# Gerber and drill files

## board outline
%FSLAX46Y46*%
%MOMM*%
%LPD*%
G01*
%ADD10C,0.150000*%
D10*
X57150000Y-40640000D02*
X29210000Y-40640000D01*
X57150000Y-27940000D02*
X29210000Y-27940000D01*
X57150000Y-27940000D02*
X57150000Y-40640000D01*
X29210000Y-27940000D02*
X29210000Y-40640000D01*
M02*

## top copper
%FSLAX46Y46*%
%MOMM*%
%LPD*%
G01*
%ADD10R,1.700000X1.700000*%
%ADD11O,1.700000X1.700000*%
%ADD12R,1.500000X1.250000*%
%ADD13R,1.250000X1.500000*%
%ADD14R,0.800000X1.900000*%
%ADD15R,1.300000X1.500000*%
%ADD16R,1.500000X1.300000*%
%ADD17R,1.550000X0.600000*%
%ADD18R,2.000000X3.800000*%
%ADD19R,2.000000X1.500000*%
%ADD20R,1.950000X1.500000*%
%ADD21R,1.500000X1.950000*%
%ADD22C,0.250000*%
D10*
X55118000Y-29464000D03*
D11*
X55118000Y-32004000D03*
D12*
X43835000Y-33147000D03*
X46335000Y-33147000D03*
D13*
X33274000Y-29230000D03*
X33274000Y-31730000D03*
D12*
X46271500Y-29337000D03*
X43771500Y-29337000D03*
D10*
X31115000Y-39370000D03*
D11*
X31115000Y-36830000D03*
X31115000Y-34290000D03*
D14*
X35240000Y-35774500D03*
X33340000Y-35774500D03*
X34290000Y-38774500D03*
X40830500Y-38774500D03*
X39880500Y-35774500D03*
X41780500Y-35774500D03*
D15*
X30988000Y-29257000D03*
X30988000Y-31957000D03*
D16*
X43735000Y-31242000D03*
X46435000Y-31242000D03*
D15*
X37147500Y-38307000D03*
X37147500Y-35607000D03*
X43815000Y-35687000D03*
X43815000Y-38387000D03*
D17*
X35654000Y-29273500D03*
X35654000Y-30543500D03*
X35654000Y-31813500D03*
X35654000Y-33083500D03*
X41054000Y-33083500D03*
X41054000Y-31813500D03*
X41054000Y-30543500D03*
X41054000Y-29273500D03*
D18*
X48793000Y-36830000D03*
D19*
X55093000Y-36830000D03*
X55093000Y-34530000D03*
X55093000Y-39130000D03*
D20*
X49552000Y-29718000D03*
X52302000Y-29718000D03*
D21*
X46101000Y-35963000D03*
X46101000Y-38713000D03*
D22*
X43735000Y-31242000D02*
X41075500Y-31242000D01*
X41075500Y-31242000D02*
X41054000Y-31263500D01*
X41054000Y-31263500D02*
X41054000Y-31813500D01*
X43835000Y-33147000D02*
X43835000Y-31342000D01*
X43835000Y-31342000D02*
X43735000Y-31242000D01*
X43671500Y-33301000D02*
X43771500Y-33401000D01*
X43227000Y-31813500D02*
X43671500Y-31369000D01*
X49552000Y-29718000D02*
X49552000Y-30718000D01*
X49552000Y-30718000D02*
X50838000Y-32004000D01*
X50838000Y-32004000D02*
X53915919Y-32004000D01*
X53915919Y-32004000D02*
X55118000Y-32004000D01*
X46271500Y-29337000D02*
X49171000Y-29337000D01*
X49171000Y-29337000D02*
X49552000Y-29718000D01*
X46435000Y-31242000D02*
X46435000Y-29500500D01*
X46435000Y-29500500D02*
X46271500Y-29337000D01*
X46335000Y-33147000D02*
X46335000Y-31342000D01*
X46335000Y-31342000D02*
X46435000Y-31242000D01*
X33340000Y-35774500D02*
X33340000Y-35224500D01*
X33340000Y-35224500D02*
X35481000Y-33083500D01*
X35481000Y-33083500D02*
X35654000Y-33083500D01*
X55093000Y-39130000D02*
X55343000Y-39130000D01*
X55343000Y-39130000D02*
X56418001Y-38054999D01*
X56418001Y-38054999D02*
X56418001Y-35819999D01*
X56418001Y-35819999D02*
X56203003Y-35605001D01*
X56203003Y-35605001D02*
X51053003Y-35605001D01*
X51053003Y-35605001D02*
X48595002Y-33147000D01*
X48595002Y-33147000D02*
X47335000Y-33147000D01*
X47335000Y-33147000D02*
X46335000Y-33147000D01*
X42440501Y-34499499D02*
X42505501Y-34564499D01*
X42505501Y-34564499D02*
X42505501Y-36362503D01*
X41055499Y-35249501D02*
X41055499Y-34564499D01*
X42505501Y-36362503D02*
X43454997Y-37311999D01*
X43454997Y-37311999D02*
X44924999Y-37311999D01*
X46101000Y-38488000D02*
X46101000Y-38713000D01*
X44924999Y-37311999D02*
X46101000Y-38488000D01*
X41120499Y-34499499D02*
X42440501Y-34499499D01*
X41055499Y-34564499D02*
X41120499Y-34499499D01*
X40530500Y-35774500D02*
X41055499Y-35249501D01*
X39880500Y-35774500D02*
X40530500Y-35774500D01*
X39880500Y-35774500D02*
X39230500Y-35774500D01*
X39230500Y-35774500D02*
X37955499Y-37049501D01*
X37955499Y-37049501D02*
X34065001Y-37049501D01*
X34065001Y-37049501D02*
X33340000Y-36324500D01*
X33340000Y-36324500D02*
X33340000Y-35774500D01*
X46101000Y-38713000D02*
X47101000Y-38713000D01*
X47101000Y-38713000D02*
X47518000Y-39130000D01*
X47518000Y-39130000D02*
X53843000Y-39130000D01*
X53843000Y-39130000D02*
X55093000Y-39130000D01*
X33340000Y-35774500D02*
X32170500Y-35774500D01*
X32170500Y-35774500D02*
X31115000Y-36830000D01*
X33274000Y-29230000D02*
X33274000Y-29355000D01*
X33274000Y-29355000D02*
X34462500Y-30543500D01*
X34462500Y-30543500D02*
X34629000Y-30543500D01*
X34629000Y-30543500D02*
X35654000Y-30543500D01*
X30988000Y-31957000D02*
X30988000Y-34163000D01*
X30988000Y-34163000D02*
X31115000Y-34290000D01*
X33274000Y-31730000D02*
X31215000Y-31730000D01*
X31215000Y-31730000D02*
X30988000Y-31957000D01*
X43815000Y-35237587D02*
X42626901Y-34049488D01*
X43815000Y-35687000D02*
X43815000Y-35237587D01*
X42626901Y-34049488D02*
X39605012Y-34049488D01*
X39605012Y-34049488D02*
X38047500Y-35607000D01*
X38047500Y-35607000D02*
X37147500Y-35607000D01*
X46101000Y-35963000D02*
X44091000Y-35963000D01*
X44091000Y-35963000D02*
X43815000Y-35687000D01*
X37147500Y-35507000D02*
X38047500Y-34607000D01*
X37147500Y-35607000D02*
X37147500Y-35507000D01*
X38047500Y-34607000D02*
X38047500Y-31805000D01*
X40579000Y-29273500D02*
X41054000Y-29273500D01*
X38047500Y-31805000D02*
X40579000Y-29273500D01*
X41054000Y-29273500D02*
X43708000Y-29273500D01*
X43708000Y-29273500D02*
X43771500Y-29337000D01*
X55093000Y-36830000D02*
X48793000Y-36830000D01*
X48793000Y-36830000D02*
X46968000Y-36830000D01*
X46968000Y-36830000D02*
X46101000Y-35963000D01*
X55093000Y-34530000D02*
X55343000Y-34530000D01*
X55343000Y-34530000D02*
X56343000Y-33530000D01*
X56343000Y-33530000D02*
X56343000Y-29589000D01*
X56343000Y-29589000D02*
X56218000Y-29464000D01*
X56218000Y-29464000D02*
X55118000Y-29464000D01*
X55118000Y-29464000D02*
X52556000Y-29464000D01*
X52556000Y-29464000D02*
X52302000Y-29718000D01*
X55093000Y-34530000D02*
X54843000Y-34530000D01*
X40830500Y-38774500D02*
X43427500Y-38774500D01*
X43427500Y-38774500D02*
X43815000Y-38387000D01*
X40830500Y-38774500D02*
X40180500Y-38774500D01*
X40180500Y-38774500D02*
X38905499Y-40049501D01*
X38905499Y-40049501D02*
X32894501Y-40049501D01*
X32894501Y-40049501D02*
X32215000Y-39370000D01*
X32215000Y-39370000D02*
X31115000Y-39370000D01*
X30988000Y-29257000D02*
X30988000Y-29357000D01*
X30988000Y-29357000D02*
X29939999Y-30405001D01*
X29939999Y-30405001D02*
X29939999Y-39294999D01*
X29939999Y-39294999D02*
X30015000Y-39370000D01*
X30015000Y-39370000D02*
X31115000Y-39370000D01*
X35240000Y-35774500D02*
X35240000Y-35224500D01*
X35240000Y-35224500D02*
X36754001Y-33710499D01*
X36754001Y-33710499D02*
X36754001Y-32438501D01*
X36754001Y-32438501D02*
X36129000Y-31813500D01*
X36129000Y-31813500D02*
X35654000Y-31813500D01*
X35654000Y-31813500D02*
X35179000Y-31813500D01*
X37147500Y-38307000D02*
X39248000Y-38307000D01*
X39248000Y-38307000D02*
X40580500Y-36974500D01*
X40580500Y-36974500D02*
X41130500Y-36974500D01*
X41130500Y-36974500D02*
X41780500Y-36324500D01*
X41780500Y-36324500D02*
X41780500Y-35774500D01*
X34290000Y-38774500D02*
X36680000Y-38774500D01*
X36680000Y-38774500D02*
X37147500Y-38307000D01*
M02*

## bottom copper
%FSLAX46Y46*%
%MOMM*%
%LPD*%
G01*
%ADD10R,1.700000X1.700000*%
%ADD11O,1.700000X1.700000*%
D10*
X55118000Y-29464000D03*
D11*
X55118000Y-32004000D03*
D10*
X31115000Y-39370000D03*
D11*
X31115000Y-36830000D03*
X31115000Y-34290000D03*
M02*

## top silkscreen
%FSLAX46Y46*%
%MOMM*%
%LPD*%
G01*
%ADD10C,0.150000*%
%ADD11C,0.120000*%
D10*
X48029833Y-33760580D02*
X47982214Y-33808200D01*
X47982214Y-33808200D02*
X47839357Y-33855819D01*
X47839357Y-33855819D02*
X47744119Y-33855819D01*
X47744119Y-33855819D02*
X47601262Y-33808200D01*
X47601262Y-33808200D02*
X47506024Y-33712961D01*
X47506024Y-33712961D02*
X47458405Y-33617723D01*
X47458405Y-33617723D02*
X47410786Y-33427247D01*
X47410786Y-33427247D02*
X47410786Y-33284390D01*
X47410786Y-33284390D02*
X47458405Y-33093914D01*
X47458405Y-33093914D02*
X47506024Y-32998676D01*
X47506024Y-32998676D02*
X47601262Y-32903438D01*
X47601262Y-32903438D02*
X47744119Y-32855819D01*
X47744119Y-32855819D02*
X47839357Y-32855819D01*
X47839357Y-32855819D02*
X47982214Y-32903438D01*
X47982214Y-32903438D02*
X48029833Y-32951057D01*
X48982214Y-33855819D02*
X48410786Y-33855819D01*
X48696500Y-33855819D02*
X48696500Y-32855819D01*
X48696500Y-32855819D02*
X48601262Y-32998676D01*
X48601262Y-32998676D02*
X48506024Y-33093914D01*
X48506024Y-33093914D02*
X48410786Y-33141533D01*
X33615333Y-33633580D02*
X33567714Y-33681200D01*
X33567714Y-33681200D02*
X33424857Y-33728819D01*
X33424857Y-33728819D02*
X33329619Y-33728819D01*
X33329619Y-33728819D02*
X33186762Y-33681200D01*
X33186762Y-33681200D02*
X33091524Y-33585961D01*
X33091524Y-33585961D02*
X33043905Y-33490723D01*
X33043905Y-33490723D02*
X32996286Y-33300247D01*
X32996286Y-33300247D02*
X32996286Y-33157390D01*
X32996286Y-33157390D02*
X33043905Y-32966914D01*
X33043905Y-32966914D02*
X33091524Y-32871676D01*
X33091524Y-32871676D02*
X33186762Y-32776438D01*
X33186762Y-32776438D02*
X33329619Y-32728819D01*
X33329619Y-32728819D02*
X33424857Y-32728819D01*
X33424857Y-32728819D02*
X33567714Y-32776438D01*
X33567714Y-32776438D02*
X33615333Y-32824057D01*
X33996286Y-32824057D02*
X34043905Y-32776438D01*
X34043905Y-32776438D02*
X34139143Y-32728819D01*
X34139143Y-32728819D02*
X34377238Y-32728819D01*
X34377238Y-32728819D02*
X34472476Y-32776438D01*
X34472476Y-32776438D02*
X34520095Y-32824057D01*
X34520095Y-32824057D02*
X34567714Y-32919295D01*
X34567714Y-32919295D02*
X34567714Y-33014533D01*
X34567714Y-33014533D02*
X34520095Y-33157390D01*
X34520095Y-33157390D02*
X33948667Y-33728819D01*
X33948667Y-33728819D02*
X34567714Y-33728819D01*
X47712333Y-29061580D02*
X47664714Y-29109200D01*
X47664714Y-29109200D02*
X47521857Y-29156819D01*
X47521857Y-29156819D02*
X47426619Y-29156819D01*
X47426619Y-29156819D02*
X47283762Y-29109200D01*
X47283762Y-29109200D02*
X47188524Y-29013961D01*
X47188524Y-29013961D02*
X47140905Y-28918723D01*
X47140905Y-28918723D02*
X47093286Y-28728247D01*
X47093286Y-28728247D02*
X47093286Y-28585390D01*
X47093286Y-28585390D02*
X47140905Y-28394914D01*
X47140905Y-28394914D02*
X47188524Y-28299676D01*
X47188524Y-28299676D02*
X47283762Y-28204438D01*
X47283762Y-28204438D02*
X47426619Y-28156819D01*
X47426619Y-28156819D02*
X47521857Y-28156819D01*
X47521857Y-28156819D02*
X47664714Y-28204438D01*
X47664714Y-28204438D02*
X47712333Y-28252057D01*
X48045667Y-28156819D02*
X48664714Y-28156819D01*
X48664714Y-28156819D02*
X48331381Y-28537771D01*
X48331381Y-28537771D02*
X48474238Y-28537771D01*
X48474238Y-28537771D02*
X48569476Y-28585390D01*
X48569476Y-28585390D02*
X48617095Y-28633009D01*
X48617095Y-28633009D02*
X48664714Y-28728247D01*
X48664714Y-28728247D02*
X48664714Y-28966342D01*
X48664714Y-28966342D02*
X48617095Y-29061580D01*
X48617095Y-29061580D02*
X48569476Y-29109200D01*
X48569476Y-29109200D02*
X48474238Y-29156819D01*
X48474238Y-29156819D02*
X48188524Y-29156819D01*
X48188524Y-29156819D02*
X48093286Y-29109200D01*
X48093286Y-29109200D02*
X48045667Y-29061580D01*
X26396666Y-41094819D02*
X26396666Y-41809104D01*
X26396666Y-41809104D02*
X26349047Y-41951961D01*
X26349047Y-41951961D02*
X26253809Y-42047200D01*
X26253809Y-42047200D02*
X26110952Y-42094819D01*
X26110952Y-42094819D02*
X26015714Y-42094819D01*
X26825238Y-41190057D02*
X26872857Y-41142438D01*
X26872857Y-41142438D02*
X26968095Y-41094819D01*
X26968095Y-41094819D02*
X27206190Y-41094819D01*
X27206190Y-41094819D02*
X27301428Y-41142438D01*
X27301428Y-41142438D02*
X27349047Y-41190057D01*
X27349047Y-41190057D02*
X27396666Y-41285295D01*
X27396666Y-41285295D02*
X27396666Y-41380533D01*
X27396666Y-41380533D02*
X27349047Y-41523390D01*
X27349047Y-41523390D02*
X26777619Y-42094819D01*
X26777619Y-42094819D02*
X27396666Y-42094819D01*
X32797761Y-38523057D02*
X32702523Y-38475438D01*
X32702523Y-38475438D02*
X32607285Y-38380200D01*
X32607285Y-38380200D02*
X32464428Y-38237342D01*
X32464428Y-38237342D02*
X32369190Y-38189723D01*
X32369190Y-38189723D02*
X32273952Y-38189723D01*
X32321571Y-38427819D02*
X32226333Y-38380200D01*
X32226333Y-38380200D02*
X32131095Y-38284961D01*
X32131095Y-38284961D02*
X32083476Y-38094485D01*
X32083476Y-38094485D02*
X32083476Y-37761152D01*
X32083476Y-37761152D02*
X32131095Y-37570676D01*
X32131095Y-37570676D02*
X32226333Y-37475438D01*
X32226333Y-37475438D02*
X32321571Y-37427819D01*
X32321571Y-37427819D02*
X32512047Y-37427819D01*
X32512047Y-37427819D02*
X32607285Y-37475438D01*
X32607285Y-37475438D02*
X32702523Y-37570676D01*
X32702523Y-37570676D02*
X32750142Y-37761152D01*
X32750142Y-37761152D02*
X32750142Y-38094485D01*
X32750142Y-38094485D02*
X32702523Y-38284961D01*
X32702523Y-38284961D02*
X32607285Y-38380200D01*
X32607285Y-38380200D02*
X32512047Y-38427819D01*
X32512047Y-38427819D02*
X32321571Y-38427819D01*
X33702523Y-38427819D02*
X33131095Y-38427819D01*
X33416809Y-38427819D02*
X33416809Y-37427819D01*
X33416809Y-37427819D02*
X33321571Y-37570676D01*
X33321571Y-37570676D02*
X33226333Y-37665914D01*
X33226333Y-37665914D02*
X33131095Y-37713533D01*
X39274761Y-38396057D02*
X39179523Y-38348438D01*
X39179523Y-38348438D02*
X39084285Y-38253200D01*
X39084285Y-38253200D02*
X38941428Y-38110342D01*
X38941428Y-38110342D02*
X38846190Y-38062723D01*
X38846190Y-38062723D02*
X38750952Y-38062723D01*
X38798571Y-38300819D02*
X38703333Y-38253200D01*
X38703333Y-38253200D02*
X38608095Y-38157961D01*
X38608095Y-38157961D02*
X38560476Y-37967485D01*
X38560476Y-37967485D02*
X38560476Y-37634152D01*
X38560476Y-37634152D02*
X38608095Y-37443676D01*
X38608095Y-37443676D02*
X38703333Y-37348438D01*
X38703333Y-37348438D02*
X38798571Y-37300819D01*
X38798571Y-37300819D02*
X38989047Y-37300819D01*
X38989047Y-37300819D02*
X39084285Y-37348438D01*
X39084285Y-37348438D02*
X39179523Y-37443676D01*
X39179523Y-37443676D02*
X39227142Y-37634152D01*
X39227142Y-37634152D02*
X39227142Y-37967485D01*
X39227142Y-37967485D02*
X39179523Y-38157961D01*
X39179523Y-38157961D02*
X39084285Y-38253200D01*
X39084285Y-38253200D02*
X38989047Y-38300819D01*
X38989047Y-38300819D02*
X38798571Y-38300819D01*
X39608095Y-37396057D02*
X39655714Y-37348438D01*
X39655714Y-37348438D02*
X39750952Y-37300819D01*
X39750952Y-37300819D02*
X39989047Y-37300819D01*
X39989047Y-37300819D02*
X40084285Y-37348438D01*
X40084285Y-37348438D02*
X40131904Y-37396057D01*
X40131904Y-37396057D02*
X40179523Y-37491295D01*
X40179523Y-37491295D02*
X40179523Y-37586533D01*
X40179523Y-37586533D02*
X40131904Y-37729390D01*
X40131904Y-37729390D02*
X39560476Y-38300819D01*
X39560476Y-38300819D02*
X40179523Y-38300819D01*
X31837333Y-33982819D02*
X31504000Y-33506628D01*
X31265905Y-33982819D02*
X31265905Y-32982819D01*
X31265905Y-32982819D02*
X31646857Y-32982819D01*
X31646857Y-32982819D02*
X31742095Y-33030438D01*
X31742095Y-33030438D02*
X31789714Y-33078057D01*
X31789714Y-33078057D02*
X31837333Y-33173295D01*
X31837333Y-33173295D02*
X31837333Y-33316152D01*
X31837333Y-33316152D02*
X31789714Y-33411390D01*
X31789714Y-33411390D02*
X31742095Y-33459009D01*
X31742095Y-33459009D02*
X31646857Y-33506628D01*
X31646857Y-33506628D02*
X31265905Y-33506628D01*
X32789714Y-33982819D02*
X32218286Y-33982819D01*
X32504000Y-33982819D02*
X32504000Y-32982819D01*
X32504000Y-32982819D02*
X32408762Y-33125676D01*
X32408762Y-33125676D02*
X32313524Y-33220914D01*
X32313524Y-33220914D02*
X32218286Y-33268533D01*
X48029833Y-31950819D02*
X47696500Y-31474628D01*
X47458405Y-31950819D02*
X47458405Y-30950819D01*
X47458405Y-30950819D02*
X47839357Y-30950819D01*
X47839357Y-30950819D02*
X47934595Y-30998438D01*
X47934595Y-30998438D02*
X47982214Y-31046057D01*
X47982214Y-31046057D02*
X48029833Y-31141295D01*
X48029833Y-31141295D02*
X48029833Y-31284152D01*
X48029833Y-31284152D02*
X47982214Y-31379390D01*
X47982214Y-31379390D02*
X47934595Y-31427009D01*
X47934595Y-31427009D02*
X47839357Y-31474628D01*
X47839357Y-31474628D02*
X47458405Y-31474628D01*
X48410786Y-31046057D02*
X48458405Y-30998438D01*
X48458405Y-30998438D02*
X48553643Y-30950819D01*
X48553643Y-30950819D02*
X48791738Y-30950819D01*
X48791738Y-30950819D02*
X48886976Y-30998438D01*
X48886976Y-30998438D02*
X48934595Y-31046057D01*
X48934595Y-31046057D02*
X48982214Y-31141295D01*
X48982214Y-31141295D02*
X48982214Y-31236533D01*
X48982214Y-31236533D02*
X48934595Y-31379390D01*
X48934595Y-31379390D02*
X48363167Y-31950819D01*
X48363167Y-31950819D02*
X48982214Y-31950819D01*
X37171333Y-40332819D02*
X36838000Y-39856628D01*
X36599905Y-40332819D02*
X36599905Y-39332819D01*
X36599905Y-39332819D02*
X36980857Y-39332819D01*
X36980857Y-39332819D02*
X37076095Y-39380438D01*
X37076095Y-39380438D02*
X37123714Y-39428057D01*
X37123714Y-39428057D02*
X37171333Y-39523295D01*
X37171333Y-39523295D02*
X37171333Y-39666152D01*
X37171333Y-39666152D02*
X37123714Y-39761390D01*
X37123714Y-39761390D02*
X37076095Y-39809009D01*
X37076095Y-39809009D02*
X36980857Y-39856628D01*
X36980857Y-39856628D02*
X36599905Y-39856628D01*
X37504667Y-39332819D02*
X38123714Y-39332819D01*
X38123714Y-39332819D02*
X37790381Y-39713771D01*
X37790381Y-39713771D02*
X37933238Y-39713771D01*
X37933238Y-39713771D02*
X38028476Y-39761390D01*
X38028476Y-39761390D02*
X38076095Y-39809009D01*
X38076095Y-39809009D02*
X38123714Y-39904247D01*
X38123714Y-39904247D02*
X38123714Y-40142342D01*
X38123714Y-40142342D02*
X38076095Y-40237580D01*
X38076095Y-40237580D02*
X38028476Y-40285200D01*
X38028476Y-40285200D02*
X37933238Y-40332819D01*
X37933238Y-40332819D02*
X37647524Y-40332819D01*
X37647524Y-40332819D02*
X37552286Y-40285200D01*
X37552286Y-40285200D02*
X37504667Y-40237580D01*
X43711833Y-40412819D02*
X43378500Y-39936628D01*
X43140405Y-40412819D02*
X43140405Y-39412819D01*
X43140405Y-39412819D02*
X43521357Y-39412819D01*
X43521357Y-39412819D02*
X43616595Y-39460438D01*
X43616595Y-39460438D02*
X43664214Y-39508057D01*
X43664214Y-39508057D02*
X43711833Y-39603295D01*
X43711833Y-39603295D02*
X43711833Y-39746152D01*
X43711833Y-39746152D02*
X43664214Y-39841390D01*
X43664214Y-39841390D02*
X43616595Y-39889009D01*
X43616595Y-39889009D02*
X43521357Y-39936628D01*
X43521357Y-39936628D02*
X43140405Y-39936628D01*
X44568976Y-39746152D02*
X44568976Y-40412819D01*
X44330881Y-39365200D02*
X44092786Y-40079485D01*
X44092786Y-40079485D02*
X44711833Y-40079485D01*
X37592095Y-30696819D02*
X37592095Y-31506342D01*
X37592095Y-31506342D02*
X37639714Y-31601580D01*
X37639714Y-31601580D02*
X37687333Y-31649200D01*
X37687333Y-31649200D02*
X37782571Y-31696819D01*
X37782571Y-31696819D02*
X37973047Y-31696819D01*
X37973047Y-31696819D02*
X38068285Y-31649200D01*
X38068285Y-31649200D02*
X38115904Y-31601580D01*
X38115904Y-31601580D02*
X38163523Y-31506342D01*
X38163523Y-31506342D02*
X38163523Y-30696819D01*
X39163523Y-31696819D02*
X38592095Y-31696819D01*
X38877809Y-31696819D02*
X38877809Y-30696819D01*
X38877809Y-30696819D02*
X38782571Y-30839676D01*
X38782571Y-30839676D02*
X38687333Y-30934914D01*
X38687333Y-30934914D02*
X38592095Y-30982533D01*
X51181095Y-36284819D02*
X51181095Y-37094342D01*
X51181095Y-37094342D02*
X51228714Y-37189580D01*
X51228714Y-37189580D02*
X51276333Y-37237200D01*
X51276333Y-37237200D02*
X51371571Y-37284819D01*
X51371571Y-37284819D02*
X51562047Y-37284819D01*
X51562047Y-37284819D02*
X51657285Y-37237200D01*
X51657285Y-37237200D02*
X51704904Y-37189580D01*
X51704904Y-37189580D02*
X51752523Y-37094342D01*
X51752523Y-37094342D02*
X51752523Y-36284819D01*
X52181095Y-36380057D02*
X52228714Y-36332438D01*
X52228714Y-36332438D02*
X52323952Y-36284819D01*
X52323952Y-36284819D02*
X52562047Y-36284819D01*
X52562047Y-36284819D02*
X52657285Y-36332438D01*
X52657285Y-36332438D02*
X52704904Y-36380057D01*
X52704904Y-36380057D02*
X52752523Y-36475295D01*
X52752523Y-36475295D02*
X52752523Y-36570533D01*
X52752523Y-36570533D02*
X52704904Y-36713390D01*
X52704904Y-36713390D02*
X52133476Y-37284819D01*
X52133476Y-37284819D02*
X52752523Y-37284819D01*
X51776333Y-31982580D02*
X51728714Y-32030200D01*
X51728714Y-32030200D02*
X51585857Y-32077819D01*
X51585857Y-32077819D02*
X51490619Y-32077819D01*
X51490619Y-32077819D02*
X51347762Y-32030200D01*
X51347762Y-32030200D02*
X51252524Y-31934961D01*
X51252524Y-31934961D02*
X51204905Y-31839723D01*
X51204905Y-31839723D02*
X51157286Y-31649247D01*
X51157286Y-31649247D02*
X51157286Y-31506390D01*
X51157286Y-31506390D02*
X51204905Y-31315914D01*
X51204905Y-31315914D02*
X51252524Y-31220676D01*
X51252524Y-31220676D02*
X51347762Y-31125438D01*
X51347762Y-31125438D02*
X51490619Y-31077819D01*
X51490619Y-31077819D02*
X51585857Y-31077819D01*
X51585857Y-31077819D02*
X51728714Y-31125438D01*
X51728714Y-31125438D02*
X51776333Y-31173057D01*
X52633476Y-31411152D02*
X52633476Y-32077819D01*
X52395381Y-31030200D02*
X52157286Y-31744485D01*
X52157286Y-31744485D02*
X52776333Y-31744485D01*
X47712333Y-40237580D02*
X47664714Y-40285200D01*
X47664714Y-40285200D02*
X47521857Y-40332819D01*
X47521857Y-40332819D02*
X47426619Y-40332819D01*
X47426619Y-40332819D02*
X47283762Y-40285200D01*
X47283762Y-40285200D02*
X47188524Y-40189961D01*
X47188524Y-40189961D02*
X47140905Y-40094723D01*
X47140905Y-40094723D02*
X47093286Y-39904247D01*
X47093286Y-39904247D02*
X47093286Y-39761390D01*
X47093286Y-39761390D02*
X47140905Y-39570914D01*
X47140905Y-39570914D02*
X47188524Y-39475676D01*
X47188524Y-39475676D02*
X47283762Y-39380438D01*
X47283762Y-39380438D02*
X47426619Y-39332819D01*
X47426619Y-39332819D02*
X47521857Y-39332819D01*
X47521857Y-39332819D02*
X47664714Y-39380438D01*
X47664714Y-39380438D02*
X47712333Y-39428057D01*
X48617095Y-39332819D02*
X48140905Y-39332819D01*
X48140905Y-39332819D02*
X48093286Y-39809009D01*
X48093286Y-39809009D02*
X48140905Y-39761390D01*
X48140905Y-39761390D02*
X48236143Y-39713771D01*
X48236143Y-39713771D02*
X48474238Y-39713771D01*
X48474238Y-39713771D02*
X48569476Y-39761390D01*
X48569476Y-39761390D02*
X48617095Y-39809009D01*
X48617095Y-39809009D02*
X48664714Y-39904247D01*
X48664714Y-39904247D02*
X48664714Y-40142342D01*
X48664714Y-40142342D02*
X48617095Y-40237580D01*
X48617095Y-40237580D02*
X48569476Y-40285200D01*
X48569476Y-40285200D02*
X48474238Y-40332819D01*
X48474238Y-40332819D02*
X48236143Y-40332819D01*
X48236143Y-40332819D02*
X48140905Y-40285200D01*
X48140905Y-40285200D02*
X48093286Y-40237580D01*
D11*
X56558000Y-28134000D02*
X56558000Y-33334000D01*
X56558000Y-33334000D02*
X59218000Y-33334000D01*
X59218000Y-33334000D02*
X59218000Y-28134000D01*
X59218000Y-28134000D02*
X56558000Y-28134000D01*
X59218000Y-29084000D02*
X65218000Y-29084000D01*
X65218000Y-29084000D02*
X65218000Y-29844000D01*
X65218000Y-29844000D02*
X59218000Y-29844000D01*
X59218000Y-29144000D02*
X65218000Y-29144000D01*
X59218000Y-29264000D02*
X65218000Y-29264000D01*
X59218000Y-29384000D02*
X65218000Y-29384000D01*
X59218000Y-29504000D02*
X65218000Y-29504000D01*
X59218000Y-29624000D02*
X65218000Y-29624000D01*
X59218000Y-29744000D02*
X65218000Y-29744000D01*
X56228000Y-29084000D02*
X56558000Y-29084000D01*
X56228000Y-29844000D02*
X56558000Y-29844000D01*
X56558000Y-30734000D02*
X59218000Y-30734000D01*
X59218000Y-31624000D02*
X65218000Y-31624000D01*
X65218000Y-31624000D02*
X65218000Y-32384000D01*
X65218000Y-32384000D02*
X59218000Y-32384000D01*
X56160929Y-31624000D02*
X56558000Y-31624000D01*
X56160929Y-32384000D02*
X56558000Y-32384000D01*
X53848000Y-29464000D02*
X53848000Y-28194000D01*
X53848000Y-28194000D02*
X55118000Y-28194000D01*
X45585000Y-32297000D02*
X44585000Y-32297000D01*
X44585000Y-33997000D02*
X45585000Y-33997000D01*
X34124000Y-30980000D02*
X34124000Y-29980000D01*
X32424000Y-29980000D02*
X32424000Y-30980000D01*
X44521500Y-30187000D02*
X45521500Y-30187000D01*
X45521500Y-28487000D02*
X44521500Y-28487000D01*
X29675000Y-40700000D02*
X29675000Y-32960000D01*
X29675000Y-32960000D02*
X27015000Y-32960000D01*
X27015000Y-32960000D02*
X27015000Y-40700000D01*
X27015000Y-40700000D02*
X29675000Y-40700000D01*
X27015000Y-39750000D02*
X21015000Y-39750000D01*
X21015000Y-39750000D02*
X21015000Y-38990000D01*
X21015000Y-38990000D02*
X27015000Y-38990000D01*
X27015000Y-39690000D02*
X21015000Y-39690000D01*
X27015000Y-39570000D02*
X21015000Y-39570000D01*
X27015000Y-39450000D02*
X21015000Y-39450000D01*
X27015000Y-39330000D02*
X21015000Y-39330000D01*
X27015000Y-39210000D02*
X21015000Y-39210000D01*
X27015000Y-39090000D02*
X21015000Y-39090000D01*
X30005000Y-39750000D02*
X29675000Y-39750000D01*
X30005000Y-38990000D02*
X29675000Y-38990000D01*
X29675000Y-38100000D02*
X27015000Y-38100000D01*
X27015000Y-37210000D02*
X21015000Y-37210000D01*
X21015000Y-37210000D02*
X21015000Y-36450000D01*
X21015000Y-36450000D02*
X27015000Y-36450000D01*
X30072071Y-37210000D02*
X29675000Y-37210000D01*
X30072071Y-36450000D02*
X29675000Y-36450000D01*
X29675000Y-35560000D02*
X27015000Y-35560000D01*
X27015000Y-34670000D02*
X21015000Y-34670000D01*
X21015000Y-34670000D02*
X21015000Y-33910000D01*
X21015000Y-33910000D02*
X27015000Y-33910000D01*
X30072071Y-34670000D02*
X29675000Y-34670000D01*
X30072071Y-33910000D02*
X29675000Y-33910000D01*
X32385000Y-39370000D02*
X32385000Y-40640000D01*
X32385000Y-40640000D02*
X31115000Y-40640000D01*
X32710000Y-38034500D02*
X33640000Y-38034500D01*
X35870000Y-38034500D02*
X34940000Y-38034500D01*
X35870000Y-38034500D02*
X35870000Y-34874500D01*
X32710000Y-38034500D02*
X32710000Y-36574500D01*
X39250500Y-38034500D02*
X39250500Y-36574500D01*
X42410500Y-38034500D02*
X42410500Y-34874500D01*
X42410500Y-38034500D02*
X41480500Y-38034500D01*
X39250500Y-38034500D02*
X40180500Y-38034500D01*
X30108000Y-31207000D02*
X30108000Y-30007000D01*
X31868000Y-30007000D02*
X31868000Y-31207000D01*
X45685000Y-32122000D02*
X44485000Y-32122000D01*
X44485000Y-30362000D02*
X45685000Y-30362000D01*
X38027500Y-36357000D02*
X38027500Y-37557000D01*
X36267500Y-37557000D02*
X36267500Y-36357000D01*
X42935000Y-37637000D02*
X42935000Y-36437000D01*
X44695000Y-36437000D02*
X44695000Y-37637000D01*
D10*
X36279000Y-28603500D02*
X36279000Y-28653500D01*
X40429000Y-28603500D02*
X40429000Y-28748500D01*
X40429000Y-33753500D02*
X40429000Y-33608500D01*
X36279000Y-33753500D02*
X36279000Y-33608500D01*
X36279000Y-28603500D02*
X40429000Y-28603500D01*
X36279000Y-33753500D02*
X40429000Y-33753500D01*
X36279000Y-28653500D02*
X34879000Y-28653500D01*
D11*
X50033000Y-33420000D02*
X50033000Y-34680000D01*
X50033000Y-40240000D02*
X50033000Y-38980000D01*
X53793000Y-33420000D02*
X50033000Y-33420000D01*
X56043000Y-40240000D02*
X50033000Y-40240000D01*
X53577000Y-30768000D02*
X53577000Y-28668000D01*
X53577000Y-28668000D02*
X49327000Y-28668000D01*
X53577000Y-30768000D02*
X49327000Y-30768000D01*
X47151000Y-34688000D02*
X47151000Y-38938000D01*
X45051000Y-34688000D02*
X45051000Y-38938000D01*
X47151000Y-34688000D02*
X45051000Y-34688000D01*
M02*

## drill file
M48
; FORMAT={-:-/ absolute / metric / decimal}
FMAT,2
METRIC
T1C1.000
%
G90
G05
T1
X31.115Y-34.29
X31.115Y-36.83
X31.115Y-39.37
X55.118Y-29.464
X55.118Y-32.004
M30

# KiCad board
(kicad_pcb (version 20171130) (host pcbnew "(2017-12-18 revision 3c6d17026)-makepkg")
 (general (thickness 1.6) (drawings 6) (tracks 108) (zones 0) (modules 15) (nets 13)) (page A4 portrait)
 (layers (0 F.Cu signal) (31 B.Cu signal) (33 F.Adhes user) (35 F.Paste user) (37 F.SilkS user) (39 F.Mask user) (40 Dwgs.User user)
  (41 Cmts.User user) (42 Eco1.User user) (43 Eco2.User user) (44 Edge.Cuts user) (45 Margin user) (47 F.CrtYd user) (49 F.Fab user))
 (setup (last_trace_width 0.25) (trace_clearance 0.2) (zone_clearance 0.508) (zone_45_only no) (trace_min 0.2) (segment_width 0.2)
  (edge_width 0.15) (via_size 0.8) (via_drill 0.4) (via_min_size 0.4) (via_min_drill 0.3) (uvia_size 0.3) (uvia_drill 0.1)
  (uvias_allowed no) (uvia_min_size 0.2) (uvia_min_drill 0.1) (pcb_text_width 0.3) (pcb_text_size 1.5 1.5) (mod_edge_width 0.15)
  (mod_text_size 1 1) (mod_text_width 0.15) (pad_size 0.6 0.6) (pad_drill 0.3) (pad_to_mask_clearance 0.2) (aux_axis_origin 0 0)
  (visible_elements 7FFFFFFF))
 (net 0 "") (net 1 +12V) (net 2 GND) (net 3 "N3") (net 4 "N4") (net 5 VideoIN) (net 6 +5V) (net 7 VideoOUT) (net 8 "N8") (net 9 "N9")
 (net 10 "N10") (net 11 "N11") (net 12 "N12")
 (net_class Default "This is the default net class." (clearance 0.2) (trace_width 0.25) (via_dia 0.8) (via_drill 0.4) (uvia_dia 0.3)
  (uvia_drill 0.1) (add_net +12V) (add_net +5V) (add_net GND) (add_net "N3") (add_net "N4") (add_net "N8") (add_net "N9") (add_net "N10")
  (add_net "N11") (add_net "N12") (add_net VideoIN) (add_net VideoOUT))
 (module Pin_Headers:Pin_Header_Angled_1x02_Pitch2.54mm (layer F.Cu) (at 55.118 29.464)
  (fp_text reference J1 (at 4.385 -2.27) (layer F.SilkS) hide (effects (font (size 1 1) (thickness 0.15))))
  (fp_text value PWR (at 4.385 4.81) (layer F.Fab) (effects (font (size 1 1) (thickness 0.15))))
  (fp_line (start 1.44 -1.33) (end 1.44 3.87) (layer F.SilkS) (width 0.12))
  (fp_line (start 1.44 3.87) (end 4.1 3.87) (layer F.SilkS) (width 0.12))
  (fp_line (start 4.1 3.87) (end 4.1 -1.33) (layer F.SilkS) (width 0.12))
  (fp_line (start 4.1 -1.33) (end 1.44 -1.33) (layer F.SilkS) (width 0.12))
  (fp_line (start 4.1 -0.38) (end 10.1 -0.38) (layer F.SilkS) (width 0.12))
  (fp_line (start 10.1 -0.38) (end 10.1 0.38) (layer F.SilkS) (width 0.12))
  (fp_line (start 10.1 0.38) (end 4.1 0.38) (layer F.SilkS) (width 0.12))
  (fp_line (start 4.1 -0.32) (end 10.1 -0.32) (layer F.SilkS) (width 0.12))
  (fp_line (start 4.1 -0.2) (end 10.1 -0.2) (layer F.SilkS) (width 0.12))
  (fp_line (start 4.1 -0.08) (end 10.1 -0.08) (layer F.SilkS) (width 0.12))
  (fp_line (start 4.1 0.04) (end 10.1 0.04) (layer F.SilkS) (width 0.12))
  (fp_line (start 4.1 0.16) (end 10.1 0.16) (layer F.SilkS) (width 0.12))
  (fp_line (start 4.1 0.28) (end 10.1 0.28) (layer F.SilkS) (width 0.12))
  (fp_line (start 1.11 -0.38) (end 1.44 -0.38) (layer F.SilkS) (width 0.12))
  (fp_line (start 1.11 0.38) (end 1.44 0.38) (layer F.SilkS) (width 0.12))
  (fp_line (start 1.44 1.27) (end 4.1 1.27) (layer F.SilkS) (width 0.12))
  (fp_line (start 4.1 2.16) (end 10.1 2.16) (layer F.SilkS) (width 0.12))
  (fp_line (start 10.1 2.16) (end 10.1 2.92) (layer F.SilkS) (width 0.12))
  (fp_line (start 10.1 2.92) (end 4.1 2.92) (layer F.SilkS) (width 0.12))
  (fp_line (start 1.042929 2.16) (end 1.44 2.16) (layer F.SilkS) (width 0.12))
  (fp_line (start 1.042929 2.92) (end 1.44 2.92) (layer F.SilkS) (width 0.12))
  (fp_line (start -1.27 0) (end -1.27 -1.27) (layer F.SilkS) (width 0.12))
  (fp_line (start -1.27 -1.27) (end 0 -1.27) (layer F.SilkS) (width 0.12))
  (pad 1 thru_hole rect (at 0 0) (size 1.7 1.7) (drill 1) (layers *.Cu *.Mask) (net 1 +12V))
  (pad 2 thru_hole oval (at 0 2.54) (size 1.7 1.7) (drill 1) (layers *.Cu *.Mask) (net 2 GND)))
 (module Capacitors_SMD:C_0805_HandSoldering (layer F.Cu) (at 45.085 33.147)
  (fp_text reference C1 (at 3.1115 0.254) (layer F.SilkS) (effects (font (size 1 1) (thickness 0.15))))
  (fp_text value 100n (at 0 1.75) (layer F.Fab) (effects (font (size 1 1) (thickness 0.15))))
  (fp_line (start 0.5 -0.85) (end -0.5 -0.85) (layer F.SilkS) (width 0.12))
  (fp_line (start -0.5 0.85) (end 0.5 0.85) (layer F.SilkS) (width 0.12))
  (pad 1 smd rect (at -1.25 0) (size 1.5 1.25) (layers F.Cu F.Paste F.Mask) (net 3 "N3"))
  (pad 2 smd rect (at 1.25 0) (size 1.5 1.25) (layers F.Cu F.Paste F.Mask) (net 2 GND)))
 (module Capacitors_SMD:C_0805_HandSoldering (layer F.Cu) (at 33.274 30.48 90)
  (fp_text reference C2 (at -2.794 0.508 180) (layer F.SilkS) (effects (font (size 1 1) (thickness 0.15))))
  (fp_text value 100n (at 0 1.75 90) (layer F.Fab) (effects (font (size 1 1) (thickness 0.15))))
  (fp_line (start -0.5 0.85) (end 0.5 0.85) (layer F.SilkS) (width 0.12))
  (fp_line (start 0.5 -0.85) (end -0.5 -0.85) (layer F.SilkS) (width 0.12))
  (pad 2 smd rect (at 1.25 0 90) (size 1.5 1.25) (layers F.Cu F.Paste F.Mask) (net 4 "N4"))
  (pad 1 smd rect (at -1.25 0 90) (size 1.5 1.25) (layers F.Cu F.Paste F.Mask) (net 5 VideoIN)))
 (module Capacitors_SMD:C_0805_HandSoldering (layer F.Cu) (at 45.0215 29.337 180)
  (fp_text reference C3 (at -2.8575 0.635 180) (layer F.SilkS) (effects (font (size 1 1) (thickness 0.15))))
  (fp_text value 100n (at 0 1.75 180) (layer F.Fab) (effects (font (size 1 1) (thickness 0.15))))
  (fp_line (start 0.5 -0.85) (end -0.5 -0.85) (layer F.SilkS) (width 0.12))
  (fp_line (start -0.5 0.85) (end 0.5 0.85) (layer F.SilkS) (width 0.12))
  (pad 1 smd rect (at -1.25 0 180) (size 1.5 1.25) (layers F.Cu F.Paste F.Mask) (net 2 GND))
  (pad 2 smd rect (at 1.25 0 180) (size 1.5 1.25) (layers F.Cu F.Paste F.Mask) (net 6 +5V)))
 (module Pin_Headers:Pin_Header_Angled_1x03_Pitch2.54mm (layer F.Cu) (at 31.115 39.37 180)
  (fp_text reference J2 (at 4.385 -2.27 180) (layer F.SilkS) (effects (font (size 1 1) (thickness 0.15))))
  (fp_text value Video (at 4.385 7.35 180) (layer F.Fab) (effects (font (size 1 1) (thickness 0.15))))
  (fp_line (start 1.44 -1.33) (end 1.44 6.41) (layer F.SilkS) (width 0.12))
  (fp_line (start 1.44 6.41) (end 4.1 6.41) (layer F.SilkS) (width 0.12))
  (fp_line (start 4.1 6.41) (end 4.1 -1.33) (layer F.SilkS) (width 0.12))
  (fp_line (start 4.1 -1.33) (end 1.44 -1.33) (layer F.SilkS) (width 0.12))
  (fp_line (start 4.1 -0.38) (end 10.1 -0.38) (layer F.SilkS) (width 0.12))
  (fp_line (start 10.1 -0.38) (end 10.1 0.38) (layer F.SilkS) (width 0.12))
  (fp_line (start 10.1 0.38) (end 4.1 0.38) (layer F.SilkS) (width 0.12))
  (fp_line (start 4.1 -0.32) (end 10.1 -0.32) (layer F.SilkS) (width 0.12))
  (fp_line (start 4.1 -0.2) (end 10.1 -0.2) (layer F.SilkS) (width 0.12))
  (fp_line (start 4.1 -0.08) (end 10.1 -0.08) (layer F.SilkS) (width 0.12))
  (fp_line (start 4.1 0.04) (end 10.1 0.04) (layer F.SilkS) (width 0.12))
  (fp_line (start 4.1 0.16) (end 10.1 0.16) (layer F.SilkS) (width 0.12))
  (fp_line (start 4.1 0.28) (end 10.1 0.28) (layer F.SilkS) (width 0.12))
  (fp_line (start 1.11 -0.38) (end 1.44 -0.38) (layer F.SilkS) (width 0.12))
  (fp_line (start 1.11 0.38) (end 1.44 0.38) (layer F.SilkS) (width 0.12))
  (fp_line (start 1.44 1.27) (end 4.1 1.27) (layer F.SilkS) (width 0.12))
  (fp_line (start 4.1 2.16) (end 10.1 2.16) (layer F.SilkS) (width 0.12))
  (fp_line (start 10.1 2.16) (end 10.1 2.92) (layer F.SilkS) (width 0.12))
  (fp_line (start 10.1 2.92) (end 4.1 2.92) (layer F.SilkS) (width 0.12))
  (fp_line (start 1.042929 2.16) (end 1.44 2.16) (layer F.SilkS) (width 0.12))
  (fp_line (start 1.042929 2.92) (end 1.44 2.92) (layer F.SilkS) (width 0.12))
  (fp_line (start 1.44 3.81) (end 4.1 3.81) (layer F.SilkS) (width 0.12))
  (fp_line (start 4.1 4.7) (end 10.1 4.7) (layer F.SilkS) (width 0.12))
  (fp_line (start 10.1 4.7) (end 10.1 5.46) (layer F.SilkS) (width 0.12))
  (fp_line (start 10.1 5.46) (end 4.1 5.46) (layer F.SilkS) (width 0.12))
  (fp_line (start 1.042929 4.7) (end 1.44 4.7) (layer F.SilkS) (width 0.12))
  (fp_line (start 1.042929 5.46) (end 1.44 5.46) (layer F.SilkS) (width 0.12))
  (fp_line (start -1.27 0) (end -1.27 -1.27) (layer F.SilkS) (width 0.12))
  (fp_line (start -1.27 -1.27) (end 0 -1.27) (layer F.SilkS) (width 0.12))
  (pad 1 thru_hole rect (at 0 0 180) (size 1.7 1.7) (drill 1) (layers *.Cu *.Mask) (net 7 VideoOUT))
  (pad 2 thru_hole oval (at 0 2.54 180) (size 1.7 1.7) (drill 1) (layers *.Cu *.Mask) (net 2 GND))
  (pad 3 thru_hole oval (at 0 5.08 180) (size 1.7 1.7) (drill 1) (layers *.Cu *.Mask) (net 5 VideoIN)))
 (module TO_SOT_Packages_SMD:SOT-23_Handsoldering (layer F.Cu) (at 34.29 37.2745 270)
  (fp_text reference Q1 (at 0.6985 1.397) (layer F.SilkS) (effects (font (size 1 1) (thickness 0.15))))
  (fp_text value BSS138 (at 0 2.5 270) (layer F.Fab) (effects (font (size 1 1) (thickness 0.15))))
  (fp_line (start 0.76 1.58) (end 0.76 0.65) (layer F.SilkS) (width 0.12))
  (fp_line (start 0.76 -1.58) (end 0.76 -0.65) (layer F.SilkS) (width 0.12))
  (fp_line (start 0.76 -1.58) (end -2.4 -1.58) (layer F.SilkS) (width 0.12))
  (fp_line (start 0.76 1.58) (end -0.7 1.58) (layer F.SilkS) (width 0.12))
  (pad 1 smd rect (at -1.5 -0.95 270) (size 1.9 0.8) (layers F.Cu F.Paste F.Mask) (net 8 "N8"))
  (pad 2 smd rect (at -1.5 0.95 270) (size 1.9 0.8) (layers F.Cu F.Paste F.Mask) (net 2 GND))
  (pad 3 smd rect (at 1.5 0 270) (size 1.9 0.8) (layers F.Cu F.Paste F.Mask) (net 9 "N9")))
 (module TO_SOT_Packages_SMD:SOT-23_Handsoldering (layer F.Cu) (at 40.8305 37.2745 270)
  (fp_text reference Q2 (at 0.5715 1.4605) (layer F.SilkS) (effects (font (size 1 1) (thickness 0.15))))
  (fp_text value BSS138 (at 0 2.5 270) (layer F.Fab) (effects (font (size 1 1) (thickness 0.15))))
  (fp_line (start 0.76 1.58) (end -0.7 1.58) (layer F.SilkS) (width 0.12))
  (fp_line (start 0.76 -1.58) (end -2.4 -1.58) (layer F.SilkS) (width 0.12))
  (fp_line (start 0.76 -1.58) (end 0.76 -0.65) (layer F.SilkS) (width 0.12))
  (fp_line (start 0.76 1.58) (end 0.76 0.65) (layer F.SilkS) (width 0.12))
  (pad 3 smd rect (at 1.5 0 270) (size 1.9 0.8) (layers F.Cu F.Paste F.Mask) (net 7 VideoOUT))
  (pad 2 smd rect (at -1.5 0.95 270) (size 1.9 0.8) (layers F.Cu F.Paste F.Mask) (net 2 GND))
  (pad 1 smd rect (at -1.5 -0.95 270) (size 1.9 0.8) (layers F.Cu F.Paste F.Mask) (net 9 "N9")))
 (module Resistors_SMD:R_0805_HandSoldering (layer F.Cu) (at 30.988 30.607 90)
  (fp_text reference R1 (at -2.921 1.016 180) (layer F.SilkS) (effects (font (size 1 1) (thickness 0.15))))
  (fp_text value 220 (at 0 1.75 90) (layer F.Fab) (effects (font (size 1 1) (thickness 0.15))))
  (fp_line (start -0.6 -0.88) (end 0.6 -0.88) (layer F.SilkS) (width 0.12))
  (fp_line (start 0.6 0.88) (end -0.6 0.88) (layer F.SilkS) (width 0.12))
  (pad 2 smd rect (at 1.35 0 90) (size 1.5 1.3) (layers F.Cu F.Paste F.Mask) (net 7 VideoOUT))
  (pad 1 smd rect (at -1.35 0 90) (size 1.5 1.3) (layers F.Cu F.Paste F.Mask) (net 5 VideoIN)))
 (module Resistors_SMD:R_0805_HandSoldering (layer F.Cu) (at 45.085 31.242)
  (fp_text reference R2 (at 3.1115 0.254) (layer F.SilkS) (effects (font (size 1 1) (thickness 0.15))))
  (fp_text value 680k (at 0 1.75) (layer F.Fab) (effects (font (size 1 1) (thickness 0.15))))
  (fp_line (start 0.6 0.88) (end -0.6 0.88) (layer F.SilkS) (width 0.12))
  (fp_line (start -0.6 -0.88) (end 0.6 -0.88) (layer F.SilkS) (width 0.12))
  (pad 1 smd rect (at -1.35 0) (size 1.5 1.3) (layers F.Cu F.Paste F.Mask) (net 3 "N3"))
  (pad 2 smd rect (at 1.35 0) (size 1.5 1.3) (layers F.Cu F.Paste F.Mask) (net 2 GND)))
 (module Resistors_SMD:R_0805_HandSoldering (layer F.Cu) (at 37.1475 36.957 270)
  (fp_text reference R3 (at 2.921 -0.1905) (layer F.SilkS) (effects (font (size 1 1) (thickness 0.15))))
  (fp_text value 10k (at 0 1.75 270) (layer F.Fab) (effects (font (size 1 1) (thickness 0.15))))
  (fp_line (start -0.6 -0.88) (end 0.6 -0.88) (layer F.SilkS) (width 0.12))
  (fp_line (start 0.6 0.88) (end -0.6 0.88) (layer F.SilkS) (width 0.12))
  (pad 2 smd rect (at 1.35 0 270) (size 1.5 1.3) (layers F.Cu F.Paste F.Mask) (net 9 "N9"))
  (pad 1 smd rect (at -1.35 0 270) (size 1.5 1.3) (layers F.Cu F.Paste F.Mask) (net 6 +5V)))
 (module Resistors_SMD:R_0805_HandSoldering (layer F.Cu) (at 43.815 37.037 270)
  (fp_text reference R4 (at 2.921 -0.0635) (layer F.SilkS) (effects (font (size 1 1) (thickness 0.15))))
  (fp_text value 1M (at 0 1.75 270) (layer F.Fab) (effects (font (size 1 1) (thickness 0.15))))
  (fp_line (start 0.6 0.88) (end -0.6 0.88) (layer F.SilkS) (width 0.12))
  (fp_line (start -0.6 -0.88) (end 0.6 -0.88) (layer F.SilkS) (width 0.12))
  (pad 1 smd rect (at -1.35 0 270) (size 1.5 1.3) (layers F.Cu F.Paste F.Mask) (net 6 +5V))
  (pad 2 smd rect (at 1.35 0 270) (size 1.5 1.3) (layers F.Cu F.Paste F.Mask) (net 7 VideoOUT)))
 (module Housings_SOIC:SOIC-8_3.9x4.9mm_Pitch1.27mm (layer F.Cu) (at 38.354 31.1785)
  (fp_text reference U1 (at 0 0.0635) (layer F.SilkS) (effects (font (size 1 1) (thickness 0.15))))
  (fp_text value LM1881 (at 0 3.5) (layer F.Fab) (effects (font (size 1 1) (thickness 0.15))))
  (fp_line (start -2.075 -2.575) (end -2.075 -2.525) (layer F.SilkS) (width 0.15))
  (fp_line (start 2.075 -2.575) (end 2.075 -2.43) (layer F.SilkS) (width 0.15))
  (fp_line (start 2.075 2.575) (end 2.075 2.43) (layer F.SilkS) (width 0.15))
  (fp_line (start -2.075 2.575) (end -2.075 2.43) (layer F.SilkS) (width 0.15))
  (fp_line (start -2.075 -2.575) (end 2.075 -2.575) (layer F.SilkS) (width 0.15))
  (fp_line (start -2.075 2.575) (end 2.075 2.575) (layer F.SilkS) (width 0.15))
  (fp_line (start -2.075 -2.525) (end -3.475 -2.525) (layer F.SilkS) (width 0.15))
  (pad 1 smd rect (at -2.7 -1.905) (size 1.55 0.6) (layers F.Cu F.Paste F.Mask) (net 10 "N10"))
  (pad 2 smd rect (at -2.7 -0.635) (size 1.55 0.6) (layers F.Cu F.Paste F.Mask) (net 4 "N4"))
  (pad 3 smd rect (at -2.7 0.635) (size 1.55 0.6) (layers F.Cu F.Paste F.Mask) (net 8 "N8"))
  (pad 4 smd rect (at -2.7 1.905) (size 1.55 0.6) (layers F.Cu F.Paste F.Mask) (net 2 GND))
  (pad 5 smd rect (at 2.7 1.905) (size 1.55 0.6) (layers F.Cu F.Paste F.Mask) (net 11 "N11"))
  (pad 6 smd rect (at 2.7 0.635) (size 1.55 0.6) (layers F.Cu F.Paste F.Mask) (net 3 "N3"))
  (pad 7 smd rect (at 2.7 -0.635) (size 1.55 0.6) (layers F.Cu F.Paste F.Mask) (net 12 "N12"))
  (pad 8 smd rect (at 2.7 -1.905) (size 1.55 0.6) (layers F.Cu F.Paste F.Mask) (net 6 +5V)))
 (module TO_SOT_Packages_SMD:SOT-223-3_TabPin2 (layer F.Cu) (at 51.943 36.83 180)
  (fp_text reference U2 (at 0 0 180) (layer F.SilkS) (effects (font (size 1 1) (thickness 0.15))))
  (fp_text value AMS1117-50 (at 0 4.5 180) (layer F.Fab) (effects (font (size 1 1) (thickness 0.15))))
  (fp_line (start 1.91 3.41) (end 1.91 2.15) (layer F.SilkS) (width 0.12))
  (fp_line (start 1.91 -3.41) (end 1.91 -2.15) (layer F.SilkS) (width 0.12))
  (fp_line (start -1.85 3.41) (end 1.91 3.41) (layer F.SilkS) (width 0.12))
  (fp_line (start -4.1 -3.41) (end 1.91 -3.41) (layer F.SilkS) (width 0.12))
  (pad 2 smd rect (at 3.15 0 180) (size 2 3.8) (layers F.Cu F.Paste F.Mask) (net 6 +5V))
  (pad 2 smd rect (at -3.15 0 180) (size 2 1.5) (layers F.Cu F.Paste F.Mask) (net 6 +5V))
  (pad 3 smd rect (at -3.15 2.3 180) (size 2 1.5) (layers F.Cu F.Paste F.Mask) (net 1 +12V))
  (pad 1 smd rect (at -3.15 -2.3 180) (size 2 1.5) (layers F.Cu F.Paste F.Mask) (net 2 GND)))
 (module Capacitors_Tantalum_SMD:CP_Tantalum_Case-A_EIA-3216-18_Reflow (layer F.Cu) (at 50.927 29.718 180)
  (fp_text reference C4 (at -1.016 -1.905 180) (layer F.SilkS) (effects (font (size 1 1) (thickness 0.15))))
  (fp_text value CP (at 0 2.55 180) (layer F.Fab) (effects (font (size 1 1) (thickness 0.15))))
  (fp_line (start -2.65 -1.05) (end -2.65 1.05) (layer F.SilkS) (width 0.12))
  (fp_line (start -2.65 1.05) (end 1.6 1.05) (layer F.SilkS) (width 0.12))
  (fp_line (start -2.65 -1.05) (end 1.6 -1.05) (layer F.SilkS) (width 0.12))
  (pad 2 smd rect (at 1.375 0 180) (size 1.95 1.5) (layers F.Cu F.Paste F.Mask) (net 2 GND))
  (pad 1 smd rect (at -1.375 0 180) (size 1.95 1.5) (layers F.Cu F.Paste F.Mask) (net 1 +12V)))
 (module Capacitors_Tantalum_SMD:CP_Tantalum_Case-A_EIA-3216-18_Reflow (layer F.Cu) (at 46.101 37.338 270)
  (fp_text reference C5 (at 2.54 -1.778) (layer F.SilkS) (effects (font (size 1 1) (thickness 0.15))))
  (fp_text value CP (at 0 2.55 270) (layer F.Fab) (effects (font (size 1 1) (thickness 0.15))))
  (fp_line (start -2.65 -1.05) (end 1.6 -1.05) (layer F.SilkS) (width 0.12))
  (fp_line (start -2.65 1.05) (end 1.6 1.05) (layer F.SilkS) (width 0.12))
  (fp_line (start -2.65 -1.05) (end -2.65 1.05) (layer F.SilkS) (width 0.12))
  (pad 1 smd rect (at -1.375 0 270) (size 1.95 1.5) (layers F.Cu F.Paste F.Mask) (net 6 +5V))
  (pad 2 smd rect (at 1.375 0 270) (size 1.95 1.5) (layers F.Cu F.Paste F.Mask) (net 2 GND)))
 (gr_line (start 57.15 40.64) (end 29.21 40.64) (angle 90) (layer Edge.Cuts) (width 0.15))
 (gr_line (start 57.15 27.94) (end 29.21 27.94) (angle 90) (layer Edge.Cuts) (width 0.15))
 (gr_line (start 57.15 27.94) (end 57.15 40.64) (angle 90) (layer Edge.Cuts) (width 0.15))
 (gr_line (start 29.21 27.94) (end 29.21 40.64) (angle 90) (layer Edge.Cuts) (width 0.15))
 (segment (start 43.735 31.242) (end 41.0755 31.242) (width 0.25) (layer F.Cu) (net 3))
 (segment (start 41.0755 31.242) (end 41.054 31.2635) (width 0.25) (layer F.Cu) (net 3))
 (segment (start 41.054 31.2635) (end 41.054 31.8135) (width 0.25) (layer F.Cu) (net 3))
 (segment (start 43.835 33.147) (end 43.835 31.342) (width 0.25) (layer F.Cu) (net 3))
 (segment (start 43.835 31.342) (end 43.735 31.242) (width 0.25) (layer F.Cu) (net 3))
 (segment (start 43.6715 33.301) (end 43.7715 33.401) (width 0.25) (layer F.Cu) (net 3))
 (segment (start 43.227 31.8135) (end 43.6715 31.369) (width 0.25) (layer F.Cu) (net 3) (status 30))
 (segment (start 49.552 29.718) (end 49.552 30.718) (width 0.25) (layer F.Cu) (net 2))
 (segment (start 49.552 30.718) (end 50.838 32.004) (width 0.25) (layer F.Cu) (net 2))
 (segment (start 50.838 32.004) (end 53.915919 32.004) (width 0.25) (layer F.Cu) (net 2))
 (segment (start 53.915919 32.004) (end 55.118 32.004) (width 0.25) (layer F.Cu) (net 2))
 (segment (start 46.2715 29.337) (end 49.171 29.337) (width 0.25) (layer F.Cu) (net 2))
 (segment (start 49.171 29.337) (end 49.552 29.718) (width 0.25) (layer F.Cu) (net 2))
 (segment (start 46.435 31.242) (end 46.435 29.5005) (width 0.25) (layer F.Cu) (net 2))
 (segment (start 46.435 29.5005) (end 46.2715 29.337) (width 0.25) (layer F.Cu) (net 2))
 (segment (start 46.335 33.147) (end 46.335 31.342) (width 0.25) (layer F.Cu) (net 2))
 (segment (start 46.335 31.342) (end 46.435 31.242) (width 0.25) (layer F.Cu) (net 2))
 (segment (start 33.34 35.7745) (end 33.34 35.2245) (width 0.25) (layer F.Cu) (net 2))
 (segment (start 33.34 35.2245) (end 35.481 33.0835) (width 0.25) (layer F.Cu) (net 2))
 (segment (start 35.481 33.0835) (end 35.654 33.0835) (width 0.25) (layer F.Cu) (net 2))
 (segment (start 55.093 39.13) (end 55.343 39.13) (width 0.25) (layer F.Cu) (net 2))
 (segment (start 55.343 39.13) (end 56.418001 38.054999) (width 0.25) (layer F.Cu) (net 2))
 (segment (start 56.418001 38.054999) (end 56.418001 35.819999) (width 0.25) (layer F.Cu) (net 2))
 (segment (start 56.418001 35.819999) (end 56.203003 35.605001) (width 0.25) (layer F.Cu) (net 2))
 (segment (start 56.203003 35.605001) (end 51.053003 35.605001) (width 0.25) (layer F.Cu) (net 2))
 (segment (start 51.053003 35.605001) (end 48.595002 33.147) (width 0.25) (layer F.Cu) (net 2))
 (segment (start 48.595002 33.147) (end 47.335 33.147) (width 0.25) (layer F.Cu) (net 2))
 (segment (start 47.335 33.147) (end 46.335 33.147) (width 0.25) (layer F.Cu) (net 2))
 (segment (start 42.440501 34.499499) (end 42.505501 34.564499) (width 0.25) (layer F.Cu) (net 2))
 (segment (start 42.505501 34.564499) (end 42.505501 36.362503) (width 0.25) (layer F.Cu) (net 2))
 (segment (start 41.055499 35.249501) (end 41.055499 34.564499) (width 0.25) (layer F.Cu) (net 2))
 (segment (start 42.505501 36.362503) (end 43.454997 37.311999) (width 0.25) (layer F.Cu) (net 2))
 (segment (start 43.454997 37.311999) (end 44.924999 37.311999) (width 0.25) (layer F.Cu) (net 2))
 (segment (start 46.101 38.488) (end 46.101 38.713) (width 0.25) (layer F.Cu) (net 2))
 (segment (start 44.924999 37.311999) (end 46.101 38.488) (width 0.25) (layer F.Cu) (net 2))
 (segment (start 41.120499 34.499499) (end 42.440501 34.499499) (width 0.25) (layer F.Cu) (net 2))
 (segment (start 41.055499 34.564499) (end 41.120499 34.499499) (width 0.25) (layer F.Cu) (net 2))
 (segment (start 40.5305 35.7745) (end 41.055499 35.249501) (width 0.25) (layer F.Cu) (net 2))
 (segment (start 39.8805 35.7745) (end 40.5305 35.7745) (width 0.25) (layer F.Cu) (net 2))
 (segment (start 39.8805 35.7745) (end 39.2305 35.7745) (width 0.25) (layer F.Cu) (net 2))
 (segment (start 39.2305 35.7745) (end 37.955499 37.049501) (width 0.25) (layer F.Cu) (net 2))
 (segment (start 37.955499 37.049501) (end 34.065001 37.049501) (width 0.25) (layer F.Cu) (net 2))
 (segment (start 34.065001 37.049501) (end 33.34 36.3245) (width 0.25) (layer F.Cu) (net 2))
 (segment (start 33.34 36.3245) (end 33.34 35.7745) (width 0.25) (layer F.Cu) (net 2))
 (segment (start 46.101 38.713) (end 47.101 38.713) (width 0.25) (layer F.Cu) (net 2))
 (segment (start 47.101 38.713) (end 47.518 39.13) (width 0.25) (layer F.Cu) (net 2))
 (segment (start 47.518 39.13) (end 53.843 39.13) (width 0.25) (layer F.Cu) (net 2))
 (segment (start 53.843 39.13) (end 55.093 39.13) (width 0.25) (layer F.Cu) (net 2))
 (segment (start 33.34 35.7745) (end 32.1705 35.7745) (width 0.25) (layer F.Cu) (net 2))
 (segment (start 32.1705 35.7745) (end 31.115 36.83) (width 0.25) (layer F.Cu) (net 2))
 (segment (start 33.274 29.23) (end 33.274 29.355) (width 0.25) (layer F.Cu) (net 4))
 (segment (start 33.274 29.355) (end 34.4625 30.5435) (width 0.25) (layer F.Cu) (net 4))
 (segment (start 34.4625 30.5435) (end 34.629 30.5435) (width 0.25) (layer F.Cu) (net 4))
 (segment (start 34.629 30.5435) (end 35.654 30.5435) (width 0.25) (layer F.Cu) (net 4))
 (segment (start 30.988 31.957) (end 30.988 34.163) (width 0.25) (layer F.Cu) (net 5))
 (segment (start 30.988 34.163) (end 31.115 34.29) (width 0.25) (layer F.Cu) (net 5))
 (segment (start 33.274 31.73) (end 31.215 31.73) (width 0.25) (layer F.Cu) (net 5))
 (segment (start 31.215 31.73) (end 30.988 31.957) (width 0.25) (layer F.Cu) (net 5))
 (segment (start 43.815 35.237587) (end 42.626901 34.049488) (width 0.25) (layer F.Cu) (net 6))
 (segment (start 43.815 35.687) (end 43.815 35.237587) (width 0.25) (layer F.Cu) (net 6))
 (segment (start 42.626901 34.049488) (end 39.605012 34.049488) (width 0.25) (layer F.Cu) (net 6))
 (segment (start 39.605012 34.049488) (end 38.0475 35.607) (width 0.25) (layer F.Cu) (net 6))
 (segment (start 38.0475 35.607) (end 37.1475 35.607) (width 0.25) (layer F.Cu) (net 6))
 (segment (start 46.101 35.963) (end 44.091 35.963) (width 0.25) (layer F.Cu) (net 6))
 (segment (start 44.091 35.963) (end 43.815 35.687) (width 0.25) (layer F.Cu) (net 6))
 (segment (start 37.1475 35.507) (end 38.0475 34.607) (width 0.25) (layer F.Cu) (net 6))
 (segment (start 37.1475 35.607) (end 37.1475 35.507) (width 0.25) (layer F.Cu) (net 6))
 (segment (start 38.0475 34.607) (end 38.0475 31.805) (width 0.25) (layer F.Cu) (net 6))
 (segment (start 40.579 29.2735) (end 41.054 29.2735) (width 0.25) (layer F.Cu) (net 6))
 (segment (start 38.0475 31.805) (end 40.579 29.2735) (width 0.25) (layer F.Cu) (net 6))
 (segment (start 41.054 29.2735) (end 43.708 29.2735) (width 0.25) (layer F.Cu) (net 6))
 (segment (start 43.708 29.2735) (end 43.7715 29.337) (width 0.25) (layer F.Cu) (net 6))
 (segment (start 55.093 36.83) (end 48.793 36.83) (width 0.25) (layer F.Cu) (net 6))
 (segment (start 48.793 36.83) (end 46.968 36.83) (width 0.25) (layer F.Cu) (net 6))
 (segment (start 46.968 36.83) (end 46.101 35.963) (width 0.25) (layer F.Cu) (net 6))
 (segment (start 55.093 34.53) (end 55.343 34.53) (width 0.25) (layer F.Cu) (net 1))
 (segment (start 55.343 34.53) (end 56.343 33.53) (width 0.25) (layer F.Cu) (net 1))
 (segment (start 56.343 33.53) (end 56.343 29.589) (width 0.25) (layer F.Cu) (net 1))
 (segment (start 56.343 29.589) (end 56.218 29.464) (width 0.25) (layer F.Cu) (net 1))
 (segment (start 56.218 29.464) (end 55.118 29.464) (width 0.25) (layer F.Cu) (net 1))
 (segment (start 55.118 29.464) (end 52.556 29.464) (width 0.25) (layer F.Cu) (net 1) (status 20))
 (segment (start 52.556 29.464) (end 52.302 29.718) (width 0.25) (layer F.Cu) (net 1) (status 30))
 (segment (start 55.093 34.53) (end 54.843 34.53) (width 0.25) (layer F.Cu) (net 1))
 (segment (start 40.8305 38.7745) (end 43.4275 38.7745) (width 0.25) (layer F.Cu) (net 7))
 (segment (start 43.4275 38.7745) (end 43.815 38.387) (width 0.25) (layer F.Cu) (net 7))
 (segment (start 40.8305 38.7745) (end 40.1805 38.7745) (width 0.25) (layer F.Cu) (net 7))
 (segment (start 40.1805 38.7745) (end 38.905499 40.049501) (width 0.25) (layer F.Cu) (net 7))
 (segment (start 38.905499 40.049501) (end 32.894501 40.049501) (width 0.25) (layer F.Cu) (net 7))
 (segment (start 32.894501 40.049501) (end 32.215 39.37) (width 0.25) (layer F.Cu) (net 7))
 (segment (start 32.215 39.37) (end 31.115 39.37) (width 0.25) (layer F.Cu) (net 7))
 (segment (start 30.988 29.257) (end 30.988 29.357) (width 0.25) (layer F.Cu) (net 7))
 (segment (start 30.988 29.357) (end 29.939999 30.405001) (width 0.25) (layer F.Cu) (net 7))
 (segment (start 29.939999 30.405001) (end 29.939999 39.294999) (width 0.25) (layer F.Cu) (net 7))
 (segment (start 29.939999 39.294999) (end 30.015 39.37) (width 0.25) (layer F.Cu) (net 7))
 (segment (start 30.015 39.37) (end 31.115 39.37) (width 0.25) (layer F.Cu) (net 7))
 (segment (start 35.24 35.7745) (end 35.24 35.2245) (width 0.25) (layer F.Cu) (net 8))
 (segment (start 35.24 35.2245) (end 36.754001 33.710499) (width 0.25) (layer F.Cu) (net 8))
 (segment (start 36.754001 33.710499) (end 36.754001 32.438501) (width 0.25) (layer F.Cu) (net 8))
 (segment (start 36.754001 32.438501) (end 36.129 31.8135) (width 0.25) (layer F.Cu) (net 8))
 (segment (start 36.129 31.8135) (end 35.654 31.8135) (width 0.25) (layer F.Cu) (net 8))
 (segment (start 35.654 31.8135) (end 35.179 31.8135) (width 0.25) (layer F.Cu) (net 8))
 (segment (start 37.1475 38.307) (end 39.248 38.307) (width 0.25) (layer F.Cu) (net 9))
 (segment (start 39.248 38.307) (end 40.5805 36.9745) (width 0.25) (layer F.Cu) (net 9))
 (segment (start 40.5805 36.9745) (end 41.1305 36.9745) (width 0.25) (layer F.Cu) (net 9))
 (segment (start 41.1305 36.9745) (end 41.7805 36.3245) (width 0.25) (layer F.Cu) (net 9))
 (segment (start 41.7805 36.3245) (end 41.7805 35.7745) (width 0.25) (layer F.Cu) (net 9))
 (segment (start 34.29 38.7745) (end 36.68 38.7745) (width 0.25) (layer F.Cu) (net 9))
 (segment (start 36.68 38.7745) (end 37.1475 38.307) (width 0.25) (layer F.Cu) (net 9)))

